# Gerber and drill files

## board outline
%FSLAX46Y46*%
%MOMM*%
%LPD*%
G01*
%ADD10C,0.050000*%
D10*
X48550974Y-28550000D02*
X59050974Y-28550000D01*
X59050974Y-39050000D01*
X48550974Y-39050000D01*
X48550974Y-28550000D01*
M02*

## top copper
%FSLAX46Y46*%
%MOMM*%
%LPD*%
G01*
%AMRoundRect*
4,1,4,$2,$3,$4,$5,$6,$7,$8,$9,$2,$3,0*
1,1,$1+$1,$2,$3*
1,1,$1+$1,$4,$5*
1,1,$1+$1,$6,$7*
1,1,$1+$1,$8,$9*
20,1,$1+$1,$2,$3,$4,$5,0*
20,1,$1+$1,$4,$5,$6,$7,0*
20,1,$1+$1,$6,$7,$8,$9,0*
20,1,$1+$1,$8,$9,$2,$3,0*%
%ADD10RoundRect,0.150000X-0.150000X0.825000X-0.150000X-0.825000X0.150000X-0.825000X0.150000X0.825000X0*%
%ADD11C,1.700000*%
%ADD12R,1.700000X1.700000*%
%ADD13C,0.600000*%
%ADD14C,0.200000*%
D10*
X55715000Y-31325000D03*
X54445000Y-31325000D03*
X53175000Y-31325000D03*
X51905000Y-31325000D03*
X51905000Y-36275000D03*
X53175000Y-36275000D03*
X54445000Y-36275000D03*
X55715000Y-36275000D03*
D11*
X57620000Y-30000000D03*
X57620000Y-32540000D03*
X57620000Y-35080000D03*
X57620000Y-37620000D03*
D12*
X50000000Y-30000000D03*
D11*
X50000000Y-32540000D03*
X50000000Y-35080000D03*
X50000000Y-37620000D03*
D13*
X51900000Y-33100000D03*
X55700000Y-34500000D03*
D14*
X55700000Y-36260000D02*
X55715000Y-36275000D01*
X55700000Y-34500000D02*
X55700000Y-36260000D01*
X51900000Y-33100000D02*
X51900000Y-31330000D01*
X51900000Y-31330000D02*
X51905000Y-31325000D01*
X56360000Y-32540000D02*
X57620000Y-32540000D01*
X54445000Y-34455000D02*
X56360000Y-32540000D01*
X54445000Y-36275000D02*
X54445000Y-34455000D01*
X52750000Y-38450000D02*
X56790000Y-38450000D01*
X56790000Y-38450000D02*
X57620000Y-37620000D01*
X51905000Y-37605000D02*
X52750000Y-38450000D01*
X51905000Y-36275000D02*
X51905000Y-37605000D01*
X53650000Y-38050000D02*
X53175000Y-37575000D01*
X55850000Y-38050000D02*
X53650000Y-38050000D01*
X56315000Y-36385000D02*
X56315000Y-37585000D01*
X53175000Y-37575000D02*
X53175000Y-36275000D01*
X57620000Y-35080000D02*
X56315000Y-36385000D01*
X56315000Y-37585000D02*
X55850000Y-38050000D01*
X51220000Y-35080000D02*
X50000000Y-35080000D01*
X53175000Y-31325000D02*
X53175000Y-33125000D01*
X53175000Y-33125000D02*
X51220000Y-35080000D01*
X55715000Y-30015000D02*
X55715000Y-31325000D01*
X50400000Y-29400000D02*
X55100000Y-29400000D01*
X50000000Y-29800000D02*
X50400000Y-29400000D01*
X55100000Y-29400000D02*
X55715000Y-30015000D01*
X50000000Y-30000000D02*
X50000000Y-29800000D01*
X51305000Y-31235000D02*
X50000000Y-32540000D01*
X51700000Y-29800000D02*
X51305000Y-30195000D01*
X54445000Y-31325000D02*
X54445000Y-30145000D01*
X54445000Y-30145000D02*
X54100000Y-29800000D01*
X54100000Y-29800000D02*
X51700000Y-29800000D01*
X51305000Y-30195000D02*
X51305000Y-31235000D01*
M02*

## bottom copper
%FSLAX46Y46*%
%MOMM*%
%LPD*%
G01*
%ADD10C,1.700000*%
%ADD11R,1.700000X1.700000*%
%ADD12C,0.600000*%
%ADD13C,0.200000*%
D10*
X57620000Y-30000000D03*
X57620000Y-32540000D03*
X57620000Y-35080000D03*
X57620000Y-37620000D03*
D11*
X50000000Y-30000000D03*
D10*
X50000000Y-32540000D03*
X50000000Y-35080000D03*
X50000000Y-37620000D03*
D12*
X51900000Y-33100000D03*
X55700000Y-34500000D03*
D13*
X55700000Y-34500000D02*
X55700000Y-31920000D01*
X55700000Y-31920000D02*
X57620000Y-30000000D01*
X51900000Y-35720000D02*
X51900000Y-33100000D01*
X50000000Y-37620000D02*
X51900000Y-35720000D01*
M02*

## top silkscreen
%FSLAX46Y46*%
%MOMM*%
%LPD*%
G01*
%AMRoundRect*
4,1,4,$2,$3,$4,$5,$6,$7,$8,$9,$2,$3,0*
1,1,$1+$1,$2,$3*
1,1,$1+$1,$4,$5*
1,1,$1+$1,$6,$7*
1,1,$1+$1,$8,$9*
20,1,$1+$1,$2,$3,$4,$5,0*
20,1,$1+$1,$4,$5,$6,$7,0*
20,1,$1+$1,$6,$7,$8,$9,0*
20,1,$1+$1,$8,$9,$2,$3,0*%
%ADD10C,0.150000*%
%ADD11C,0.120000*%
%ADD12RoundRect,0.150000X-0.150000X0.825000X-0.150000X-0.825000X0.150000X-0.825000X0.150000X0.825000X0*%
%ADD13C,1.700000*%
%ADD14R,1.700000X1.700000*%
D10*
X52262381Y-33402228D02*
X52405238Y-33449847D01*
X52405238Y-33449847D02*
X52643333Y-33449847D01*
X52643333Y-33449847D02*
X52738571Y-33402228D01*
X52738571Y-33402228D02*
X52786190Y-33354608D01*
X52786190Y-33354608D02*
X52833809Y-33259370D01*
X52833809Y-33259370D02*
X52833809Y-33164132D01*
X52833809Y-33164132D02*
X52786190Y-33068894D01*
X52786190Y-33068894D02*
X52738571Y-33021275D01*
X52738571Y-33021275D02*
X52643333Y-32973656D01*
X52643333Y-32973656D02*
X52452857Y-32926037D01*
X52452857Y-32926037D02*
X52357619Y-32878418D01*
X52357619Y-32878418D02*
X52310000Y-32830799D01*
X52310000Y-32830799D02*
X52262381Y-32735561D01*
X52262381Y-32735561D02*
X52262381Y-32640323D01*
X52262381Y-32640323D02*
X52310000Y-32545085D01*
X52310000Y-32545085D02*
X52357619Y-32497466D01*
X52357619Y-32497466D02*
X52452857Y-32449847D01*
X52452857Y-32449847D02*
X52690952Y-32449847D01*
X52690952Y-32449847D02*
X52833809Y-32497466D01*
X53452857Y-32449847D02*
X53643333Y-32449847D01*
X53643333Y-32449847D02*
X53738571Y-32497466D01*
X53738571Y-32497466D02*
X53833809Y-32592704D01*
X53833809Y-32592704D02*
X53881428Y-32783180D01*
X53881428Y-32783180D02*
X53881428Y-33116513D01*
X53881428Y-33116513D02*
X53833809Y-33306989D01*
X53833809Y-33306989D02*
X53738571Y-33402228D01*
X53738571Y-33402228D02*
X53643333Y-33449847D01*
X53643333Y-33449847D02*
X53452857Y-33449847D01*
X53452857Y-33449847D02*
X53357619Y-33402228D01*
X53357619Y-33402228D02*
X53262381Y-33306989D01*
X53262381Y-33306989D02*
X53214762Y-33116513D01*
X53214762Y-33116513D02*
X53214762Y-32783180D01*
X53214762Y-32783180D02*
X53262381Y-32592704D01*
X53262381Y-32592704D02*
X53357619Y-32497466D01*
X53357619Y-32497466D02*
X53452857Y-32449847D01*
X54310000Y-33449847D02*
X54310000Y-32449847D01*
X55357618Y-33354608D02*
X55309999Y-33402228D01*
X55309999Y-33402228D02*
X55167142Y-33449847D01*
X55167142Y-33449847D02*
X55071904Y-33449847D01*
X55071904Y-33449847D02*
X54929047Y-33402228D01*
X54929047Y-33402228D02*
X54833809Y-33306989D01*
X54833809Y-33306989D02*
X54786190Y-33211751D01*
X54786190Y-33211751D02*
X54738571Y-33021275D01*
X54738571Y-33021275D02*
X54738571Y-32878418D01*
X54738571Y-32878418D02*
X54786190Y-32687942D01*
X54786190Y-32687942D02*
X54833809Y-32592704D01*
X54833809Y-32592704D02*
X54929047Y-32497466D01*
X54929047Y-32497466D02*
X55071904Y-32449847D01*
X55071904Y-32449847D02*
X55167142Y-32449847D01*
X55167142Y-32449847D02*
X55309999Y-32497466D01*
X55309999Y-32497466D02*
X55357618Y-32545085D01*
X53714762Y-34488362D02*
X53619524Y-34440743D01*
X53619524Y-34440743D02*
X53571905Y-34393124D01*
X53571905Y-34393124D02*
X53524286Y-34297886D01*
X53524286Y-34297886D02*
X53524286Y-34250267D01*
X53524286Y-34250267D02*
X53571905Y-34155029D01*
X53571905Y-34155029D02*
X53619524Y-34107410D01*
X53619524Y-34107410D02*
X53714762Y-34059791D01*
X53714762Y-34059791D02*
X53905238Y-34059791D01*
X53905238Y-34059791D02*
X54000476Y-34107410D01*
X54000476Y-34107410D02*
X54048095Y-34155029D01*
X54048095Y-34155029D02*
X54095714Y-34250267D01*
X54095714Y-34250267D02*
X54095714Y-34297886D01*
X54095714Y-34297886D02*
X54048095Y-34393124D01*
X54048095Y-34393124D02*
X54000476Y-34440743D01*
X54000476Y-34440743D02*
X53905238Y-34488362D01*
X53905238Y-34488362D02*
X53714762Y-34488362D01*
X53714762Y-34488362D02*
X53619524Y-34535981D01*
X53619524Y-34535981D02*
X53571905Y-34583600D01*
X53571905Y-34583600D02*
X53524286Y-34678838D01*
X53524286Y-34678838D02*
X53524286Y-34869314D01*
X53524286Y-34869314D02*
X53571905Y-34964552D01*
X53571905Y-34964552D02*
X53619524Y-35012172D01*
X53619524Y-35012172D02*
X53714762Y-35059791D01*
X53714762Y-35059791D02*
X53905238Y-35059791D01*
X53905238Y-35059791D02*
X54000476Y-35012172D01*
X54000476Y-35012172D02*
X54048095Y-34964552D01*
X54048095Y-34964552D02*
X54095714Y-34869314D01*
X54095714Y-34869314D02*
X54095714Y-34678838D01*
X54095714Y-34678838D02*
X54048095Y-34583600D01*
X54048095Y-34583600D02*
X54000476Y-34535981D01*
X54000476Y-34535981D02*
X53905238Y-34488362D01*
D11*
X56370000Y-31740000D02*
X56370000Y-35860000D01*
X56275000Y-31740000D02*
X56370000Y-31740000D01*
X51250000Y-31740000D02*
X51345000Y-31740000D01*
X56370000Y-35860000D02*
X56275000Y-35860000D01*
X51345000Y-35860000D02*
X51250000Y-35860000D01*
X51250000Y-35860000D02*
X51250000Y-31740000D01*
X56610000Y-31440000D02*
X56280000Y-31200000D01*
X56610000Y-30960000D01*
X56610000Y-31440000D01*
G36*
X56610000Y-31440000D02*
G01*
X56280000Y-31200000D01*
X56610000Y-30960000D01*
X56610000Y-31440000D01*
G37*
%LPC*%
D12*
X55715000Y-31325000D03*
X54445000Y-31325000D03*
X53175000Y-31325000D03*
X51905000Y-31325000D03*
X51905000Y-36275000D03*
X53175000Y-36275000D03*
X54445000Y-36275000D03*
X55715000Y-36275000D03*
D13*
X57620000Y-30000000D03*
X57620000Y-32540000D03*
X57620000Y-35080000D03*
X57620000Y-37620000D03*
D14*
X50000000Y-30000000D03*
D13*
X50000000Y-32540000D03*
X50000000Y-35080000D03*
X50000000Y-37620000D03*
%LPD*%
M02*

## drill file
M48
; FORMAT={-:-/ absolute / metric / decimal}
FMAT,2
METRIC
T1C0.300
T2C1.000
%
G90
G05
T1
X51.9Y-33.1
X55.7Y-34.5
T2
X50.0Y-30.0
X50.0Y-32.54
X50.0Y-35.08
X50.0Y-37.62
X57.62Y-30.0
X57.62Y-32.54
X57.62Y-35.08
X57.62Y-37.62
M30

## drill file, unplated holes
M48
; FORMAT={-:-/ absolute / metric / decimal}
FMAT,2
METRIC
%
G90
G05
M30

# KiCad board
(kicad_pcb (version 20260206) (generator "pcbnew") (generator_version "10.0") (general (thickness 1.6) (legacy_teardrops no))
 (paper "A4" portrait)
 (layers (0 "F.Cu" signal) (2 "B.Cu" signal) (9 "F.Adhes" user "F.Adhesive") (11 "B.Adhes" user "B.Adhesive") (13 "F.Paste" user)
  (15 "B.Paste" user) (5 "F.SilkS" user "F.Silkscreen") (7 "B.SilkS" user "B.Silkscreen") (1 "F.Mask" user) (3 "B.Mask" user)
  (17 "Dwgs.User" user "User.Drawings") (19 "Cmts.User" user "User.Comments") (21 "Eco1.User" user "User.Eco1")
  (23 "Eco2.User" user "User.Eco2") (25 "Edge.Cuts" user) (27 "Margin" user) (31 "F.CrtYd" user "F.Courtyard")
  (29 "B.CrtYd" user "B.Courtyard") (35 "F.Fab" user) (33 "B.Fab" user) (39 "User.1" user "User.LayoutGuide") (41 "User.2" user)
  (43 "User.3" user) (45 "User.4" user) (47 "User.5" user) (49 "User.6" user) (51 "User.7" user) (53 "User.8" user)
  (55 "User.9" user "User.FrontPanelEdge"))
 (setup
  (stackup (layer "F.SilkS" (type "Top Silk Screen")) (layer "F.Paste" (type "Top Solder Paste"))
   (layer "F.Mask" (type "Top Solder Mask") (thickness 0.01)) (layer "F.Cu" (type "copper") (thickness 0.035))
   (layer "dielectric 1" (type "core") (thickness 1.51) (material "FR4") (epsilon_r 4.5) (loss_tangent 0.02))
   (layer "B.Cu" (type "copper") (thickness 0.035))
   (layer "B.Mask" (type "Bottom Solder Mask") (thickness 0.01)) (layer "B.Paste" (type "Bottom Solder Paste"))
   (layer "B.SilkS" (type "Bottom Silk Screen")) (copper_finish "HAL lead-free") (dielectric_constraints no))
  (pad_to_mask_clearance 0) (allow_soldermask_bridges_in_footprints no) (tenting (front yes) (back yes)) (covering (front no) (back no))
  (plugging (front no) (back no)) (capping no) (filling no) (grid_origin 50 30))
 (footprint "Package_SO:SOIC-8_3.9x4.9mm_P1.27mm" (layer "F.Cu") (at 53.81 33.8 -90)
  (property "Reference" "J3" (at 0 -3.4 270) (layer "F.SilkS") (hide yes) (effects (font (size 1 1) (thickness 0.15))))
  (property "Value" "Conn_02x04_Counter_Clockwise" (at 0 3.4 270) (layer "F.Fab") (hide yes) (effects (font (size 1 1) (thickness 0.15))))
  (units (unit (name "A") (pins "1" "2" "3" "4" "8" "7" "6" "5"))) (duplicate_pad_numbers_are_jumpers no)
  (fp_line (start -2.06 2.56) (end -2.06 2.465) (stroke (width 0.12) (type solid)) (layer "F.SilkS"))
  (fp_line (start 2.06 2.56) (end -2.06 2.56) (stroke (width 0.12) (type solid)) (layer "F.SilkS"))
  (fp_line (start 2.06 2.465) (end 2.06 2.56) (stroke (width 0.12) (type solid)) (layer "F.SilkS"))
  (fp_line (start -2.06 -2.465) (end -2.06 -2.56) (stroke (width 0.12) (type solid)) (layer "F.SilkS"))
  (fp_line (start -2.06 -2.56) (end 2.06 -2.56) (stroke (width 0.12) (type solid)) (layer "F.SilkS"))
  (fp_line (start 2.06 -2.56) (end 2.06 -2.465) (stroke (width 0.12) (type solid)) (layer "F.SilkS"))
  (fp_poly (pts (xy -2.6 -2.47) (xy -2.84 -2.8) (xy -2.36 -2.8)) (stroke (width 0.12) (type solid)) (fill yes) (layer "F.SilkS"))
  (pad "1" smd roundrect (at -2.475 -1.905 270) (size 1.95 0.6) (layers "F.Cu" "F.Mask" "F.Paste") (roundrect_rratio 0.25)
   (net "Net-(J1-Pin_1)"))
  (pad "2" smd roundrect (at -2.475 -0.635 270) (size 1.95 0.6) (layers "F.Cu" "F.Mask" "F.Paste") (roundrect_rratio 0.25)
   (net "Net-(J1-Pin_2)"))
  (pad "3" smd roundrect (at -2.475 0.635 270) (size 1.95 0.6) (layers "F.Cu" "F.Mask" "F.Paste") (roundrect_rratio 0.25)
   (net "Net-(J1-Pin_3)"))
  (pad "4" smd roundrect (at -2.475 1.905 270) (size 1.95 0.6) (layers "F.Cu" "F.Mask" "F.Paste") (roundrect_rratio 0.25)
   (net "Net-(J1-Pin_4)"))
  (pad "5" smd roundrect (at 2.475 1.905 270) (size 1.95 0.6) (layers "F.Cu" "F.Mask" "F.Paste") (roundrect_rratio 0.25)
   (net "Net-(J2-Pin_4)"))
  (pad "6" smd roundrect (at 2.475 0.635 270) (size 1.95 0.6) (layers "F.Cu" "F.Mask" "F.Paste") (roundrect_rratio 0.25)
   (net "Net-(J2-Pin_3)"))
  (pad "7" smd roundrect (at 2.475 -0.635 270) (size 1.95 0.6) (layers "F.Cu" "F.Mask" "F.Paste") (roundrect_rratio 0.25)
   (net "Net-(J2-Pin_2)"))
  (pad "8" smd roundrect (at 2.475 -1.905 270) (size 1.95 0.6) (layers "F.Cu" "F.Mask" "F.Paste") (roundrect_rratio 0.25)
   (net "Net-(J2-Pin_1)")))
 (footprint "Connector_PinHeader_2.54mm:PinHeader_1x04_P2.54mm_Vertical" (layer "B.Cu") (at 50 30 180)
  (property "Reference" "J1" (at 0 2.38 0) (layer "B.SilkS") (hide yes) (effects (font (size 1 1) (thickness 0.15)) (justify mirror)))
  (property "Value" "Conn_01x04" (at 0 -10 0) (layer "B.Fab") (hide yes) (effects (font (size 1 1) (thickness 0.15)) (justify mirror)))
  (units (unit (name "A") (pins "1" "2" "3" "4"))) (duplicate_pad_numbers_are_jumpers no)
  (pad "1" thru_hole rect (at 0 0 180) (size 1.7 1.7) (drill 1) (layers "*.Cu" "*.Mask") (remove_unused_layers no) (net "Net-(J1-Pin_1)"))
  (pad "2" thru_hole circle (at 0 -2.54 180) (size 1.7 1.7) (drill 1) (layers "*.Cu" "*.Mask") (remove_unused_layers no)
   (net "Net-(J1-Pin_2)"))
  (pad "3" thru_hole circle (at 0 -5.08 180) (size 1.7 1.7) (drill 1) (layers "*.Cu" "*.Mask") (remove_unused_layers no)
   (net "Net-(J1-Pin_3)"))
  (pad "4" thru_hole circle (at 0 -7.62 180) (size 1.7 1.7) (drill 1) (layers "*.Cu" "*.Mask") (remove_unused_layers no)
   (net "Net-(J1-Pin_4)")))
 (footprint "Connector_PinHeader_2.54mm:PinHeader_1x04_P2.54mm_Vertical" (layer "B.Cu") (at 57.62 30 180)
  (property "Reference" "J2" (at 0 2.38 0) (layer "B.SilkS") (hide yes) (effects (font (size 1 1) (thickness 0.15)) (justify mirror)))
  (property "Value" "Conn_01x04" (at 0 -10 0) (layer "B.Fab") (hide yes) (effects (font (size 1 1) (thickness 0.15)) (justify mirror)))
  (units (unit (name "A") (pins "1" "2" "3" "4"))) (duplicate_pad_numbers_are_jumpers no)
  (pad "1" thru_hole circle (at 0 0 180) (size 1.7 1.7) (drill 1) (layers "*.Cu" "*.Mask") (remove_unused_layers no) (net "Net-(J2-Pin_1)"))
  (pad "2" thru_hole circle (at 0 -2.54 180) (size 1.7 1.7) (drill 1) (layers "*.Cu" "*.Mask") (remove_unused_layers no)
   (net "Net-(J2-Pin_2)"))
  (pad "3" thru_hole circle (at 0 -5.08 180) (size 1.7 1.7) (drill 1) (layers "*.Cu" "*.Mask") (remove_unused_layers no)
   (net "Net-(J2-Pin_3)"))
  (pad "4" thru_hole circle (at 0 -7.62 180) (size 1.7 1.7) (drill 1) (layers "*.Cu" "*.Mask") (remove_unused_layers no)
   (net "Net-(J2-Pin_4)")))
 (gr_rect (start 48.550974 28.55) (end 59.050974 39.05) (stroke (width 0.05) (type solid)) (fill no) (layer "Edge.Cuts"))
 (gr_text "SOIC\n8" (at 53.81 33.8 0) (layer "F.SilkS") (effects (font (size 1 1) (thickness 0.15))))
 (segment (start 50 30) (end 50 29.8) (width 0.2) (layer "F.Cu") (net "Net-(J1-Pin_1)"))
 (segment (start 55.1 29.4) (end 55.715 30.015) (width 0.2) (layer "F.Cu") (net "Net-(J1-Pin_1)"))
 (segment (start 55.715 30.015) (end 55.715 31.325) (width 0.2) (layer "F.Cu") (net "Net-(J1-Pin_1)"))
 (segment (start 50.4 29.4) (end 55.1 29.4) (width 0.2) (layer "F.Cu") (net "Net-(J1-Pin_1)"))
 (segment (start 50 29.8) (end 50.4 29.4) (width 0.2) (layer "F.Cu") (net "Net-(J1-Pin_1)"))
 (segment (start 54.1 29.8) (end 51.7 29.8) (width 0.2) (layer "F.Cu") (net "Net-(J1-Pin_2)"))
 (segment (start 51.305 31.235) (end 50 32.54) (width 0.2) (layer "F.Cu") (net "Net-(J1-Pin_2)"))
 (segment (start 51.7 29.8) (end 51.305 30.195) (width 0.2) (layer "F.Cu") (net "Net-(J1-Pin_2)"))
 (segment (start 51.305 30.195) (end 51.305 31.235) (width 0.2) (layer "F.Cu") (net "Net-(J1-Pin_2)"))
 (segment (start 54.445 30.145) (end 54.1 29.8) (width 0.2) (layer "F.Cu") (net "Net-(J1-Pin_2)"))
 (segment (start 54.445 31.325) (end 54.445 30.145) (width 0.2) (layer "F.Cu") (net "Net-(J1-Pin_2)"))
 (segment (start 51.22 35.08) (end 50 35.08) (width 0.2) (layer "F.Cu") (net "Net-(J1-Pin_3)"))
 (segment (start 53.175 33.125) (end 51.22 35.08) (width 0.2) (layer "F.Cu") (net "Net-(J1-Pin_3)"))
 (segment (start 53.175 31.325) (end 53.175 33.125) (width 0.2) (layer "F.Cu") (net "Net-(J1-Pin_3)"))
 (segment (start 51.9 33.1) (end 51.9 31.33) (width 0.2) (layer "F.Cu") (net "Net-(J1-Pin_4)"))
 (segment (start 51.9 31.33) (end 51.905 31.325) (width 0.2) (layer "F.Cu") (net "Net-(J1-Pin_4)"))
 (via (at 51.9 33.1) (size 0.6) (drill 0.3) (layers "F.Cu" "B.Cu") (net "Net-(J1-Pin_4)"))
 (segment (start 51.9 35.72) (end 51.9 33.1) (width 0.2) (layer "B.Cu") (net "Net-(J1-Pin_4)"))
 (segment (start 50 37.62) (end 51.9 35.72) (width 0.2) (layer "B.Cu") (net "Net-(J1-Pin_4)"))
 (segment (start 56.79 38.45) (end 57.62 37.62) (width 0.2) (layer "F.Cu") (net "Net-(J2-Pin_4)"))
 (segment (start 51.905 37.605) (end 52.75 38.45) (width 0.2) (layer "F.Cu") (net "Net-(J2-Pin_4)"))
 (segment (start 51.905 36.275) (end 51.905 37.605) (width 0.2) (layer "F.Cu") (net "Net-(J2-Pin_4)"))
 (segment (start 52.75 38.45) (end 56.79 38.45) (width 0.2) (layer "F.Cu") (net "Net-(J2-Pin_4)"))
 (segment (start 53.65 38.05) (end 53.175 37.575) (width 0.2) (layer "F.Cu") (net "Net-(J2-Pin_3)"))
 (segment (start 55.85 38.05) (end 53.65 38.05) (width 0.2) (layer "F.Cu") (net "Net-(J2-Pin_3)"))
 (segment (start 56.315 36.385) (end 56.315 37.585) (width 0.2) (layer "F.Cu") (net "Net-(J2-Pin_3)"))
 (segment (start 57.62 35.08) (end 56.315 36.385) (width 0.2) (layer "F.Cu") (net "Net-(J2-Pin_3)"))
 (segment (start 53.175 37.575) (end 53.175 36.275) (width 0.2) (layer "F.Cu") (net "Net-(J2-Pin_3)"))
 (segment (start 56.315 37.585) (end 55.85 38.05) (width 0.2) (layer "F.Cu") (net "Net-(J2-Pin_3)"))
 (segment (start 54.445 36.275) (end 54.445 34.455) (width 0.2) (layer "F.Cu") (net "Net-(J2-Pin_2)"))
 (segment (start 54.445 34.455) (end 56.36 32.54) (width 0.2) (layer "F.Cu") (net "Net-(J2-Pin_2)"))
 (segment (start 56.36 32.54) (end 57.62 32.54) (width 0.2) (layer "F.Cu") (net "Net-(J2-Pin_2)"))
 (segment (start 55.7 34.5) (end 55.7 36.26) (width 0.2) (layer "F.Cu") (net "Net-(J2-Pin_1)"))
 (segment (start 55.7 36.26) (end 55.715 36.275) (width 0.2) (layer "F.Cu") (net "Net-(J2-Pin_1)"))
 (via (at 55.7 34.5) (size 0.6) (drill 0.3) (layers "F.Cu" "B.Cu") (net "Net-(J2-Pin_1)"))
 (segment (start 55.7 34.5) (end 55.7 31.92) (width 0.2) (layer "B.Cu") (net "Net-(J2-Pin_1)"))
 (segment (start 55.7 31.92) (end 57.62 30) (width 0.2) (layer "B.Cu") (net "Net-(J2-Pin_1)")))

